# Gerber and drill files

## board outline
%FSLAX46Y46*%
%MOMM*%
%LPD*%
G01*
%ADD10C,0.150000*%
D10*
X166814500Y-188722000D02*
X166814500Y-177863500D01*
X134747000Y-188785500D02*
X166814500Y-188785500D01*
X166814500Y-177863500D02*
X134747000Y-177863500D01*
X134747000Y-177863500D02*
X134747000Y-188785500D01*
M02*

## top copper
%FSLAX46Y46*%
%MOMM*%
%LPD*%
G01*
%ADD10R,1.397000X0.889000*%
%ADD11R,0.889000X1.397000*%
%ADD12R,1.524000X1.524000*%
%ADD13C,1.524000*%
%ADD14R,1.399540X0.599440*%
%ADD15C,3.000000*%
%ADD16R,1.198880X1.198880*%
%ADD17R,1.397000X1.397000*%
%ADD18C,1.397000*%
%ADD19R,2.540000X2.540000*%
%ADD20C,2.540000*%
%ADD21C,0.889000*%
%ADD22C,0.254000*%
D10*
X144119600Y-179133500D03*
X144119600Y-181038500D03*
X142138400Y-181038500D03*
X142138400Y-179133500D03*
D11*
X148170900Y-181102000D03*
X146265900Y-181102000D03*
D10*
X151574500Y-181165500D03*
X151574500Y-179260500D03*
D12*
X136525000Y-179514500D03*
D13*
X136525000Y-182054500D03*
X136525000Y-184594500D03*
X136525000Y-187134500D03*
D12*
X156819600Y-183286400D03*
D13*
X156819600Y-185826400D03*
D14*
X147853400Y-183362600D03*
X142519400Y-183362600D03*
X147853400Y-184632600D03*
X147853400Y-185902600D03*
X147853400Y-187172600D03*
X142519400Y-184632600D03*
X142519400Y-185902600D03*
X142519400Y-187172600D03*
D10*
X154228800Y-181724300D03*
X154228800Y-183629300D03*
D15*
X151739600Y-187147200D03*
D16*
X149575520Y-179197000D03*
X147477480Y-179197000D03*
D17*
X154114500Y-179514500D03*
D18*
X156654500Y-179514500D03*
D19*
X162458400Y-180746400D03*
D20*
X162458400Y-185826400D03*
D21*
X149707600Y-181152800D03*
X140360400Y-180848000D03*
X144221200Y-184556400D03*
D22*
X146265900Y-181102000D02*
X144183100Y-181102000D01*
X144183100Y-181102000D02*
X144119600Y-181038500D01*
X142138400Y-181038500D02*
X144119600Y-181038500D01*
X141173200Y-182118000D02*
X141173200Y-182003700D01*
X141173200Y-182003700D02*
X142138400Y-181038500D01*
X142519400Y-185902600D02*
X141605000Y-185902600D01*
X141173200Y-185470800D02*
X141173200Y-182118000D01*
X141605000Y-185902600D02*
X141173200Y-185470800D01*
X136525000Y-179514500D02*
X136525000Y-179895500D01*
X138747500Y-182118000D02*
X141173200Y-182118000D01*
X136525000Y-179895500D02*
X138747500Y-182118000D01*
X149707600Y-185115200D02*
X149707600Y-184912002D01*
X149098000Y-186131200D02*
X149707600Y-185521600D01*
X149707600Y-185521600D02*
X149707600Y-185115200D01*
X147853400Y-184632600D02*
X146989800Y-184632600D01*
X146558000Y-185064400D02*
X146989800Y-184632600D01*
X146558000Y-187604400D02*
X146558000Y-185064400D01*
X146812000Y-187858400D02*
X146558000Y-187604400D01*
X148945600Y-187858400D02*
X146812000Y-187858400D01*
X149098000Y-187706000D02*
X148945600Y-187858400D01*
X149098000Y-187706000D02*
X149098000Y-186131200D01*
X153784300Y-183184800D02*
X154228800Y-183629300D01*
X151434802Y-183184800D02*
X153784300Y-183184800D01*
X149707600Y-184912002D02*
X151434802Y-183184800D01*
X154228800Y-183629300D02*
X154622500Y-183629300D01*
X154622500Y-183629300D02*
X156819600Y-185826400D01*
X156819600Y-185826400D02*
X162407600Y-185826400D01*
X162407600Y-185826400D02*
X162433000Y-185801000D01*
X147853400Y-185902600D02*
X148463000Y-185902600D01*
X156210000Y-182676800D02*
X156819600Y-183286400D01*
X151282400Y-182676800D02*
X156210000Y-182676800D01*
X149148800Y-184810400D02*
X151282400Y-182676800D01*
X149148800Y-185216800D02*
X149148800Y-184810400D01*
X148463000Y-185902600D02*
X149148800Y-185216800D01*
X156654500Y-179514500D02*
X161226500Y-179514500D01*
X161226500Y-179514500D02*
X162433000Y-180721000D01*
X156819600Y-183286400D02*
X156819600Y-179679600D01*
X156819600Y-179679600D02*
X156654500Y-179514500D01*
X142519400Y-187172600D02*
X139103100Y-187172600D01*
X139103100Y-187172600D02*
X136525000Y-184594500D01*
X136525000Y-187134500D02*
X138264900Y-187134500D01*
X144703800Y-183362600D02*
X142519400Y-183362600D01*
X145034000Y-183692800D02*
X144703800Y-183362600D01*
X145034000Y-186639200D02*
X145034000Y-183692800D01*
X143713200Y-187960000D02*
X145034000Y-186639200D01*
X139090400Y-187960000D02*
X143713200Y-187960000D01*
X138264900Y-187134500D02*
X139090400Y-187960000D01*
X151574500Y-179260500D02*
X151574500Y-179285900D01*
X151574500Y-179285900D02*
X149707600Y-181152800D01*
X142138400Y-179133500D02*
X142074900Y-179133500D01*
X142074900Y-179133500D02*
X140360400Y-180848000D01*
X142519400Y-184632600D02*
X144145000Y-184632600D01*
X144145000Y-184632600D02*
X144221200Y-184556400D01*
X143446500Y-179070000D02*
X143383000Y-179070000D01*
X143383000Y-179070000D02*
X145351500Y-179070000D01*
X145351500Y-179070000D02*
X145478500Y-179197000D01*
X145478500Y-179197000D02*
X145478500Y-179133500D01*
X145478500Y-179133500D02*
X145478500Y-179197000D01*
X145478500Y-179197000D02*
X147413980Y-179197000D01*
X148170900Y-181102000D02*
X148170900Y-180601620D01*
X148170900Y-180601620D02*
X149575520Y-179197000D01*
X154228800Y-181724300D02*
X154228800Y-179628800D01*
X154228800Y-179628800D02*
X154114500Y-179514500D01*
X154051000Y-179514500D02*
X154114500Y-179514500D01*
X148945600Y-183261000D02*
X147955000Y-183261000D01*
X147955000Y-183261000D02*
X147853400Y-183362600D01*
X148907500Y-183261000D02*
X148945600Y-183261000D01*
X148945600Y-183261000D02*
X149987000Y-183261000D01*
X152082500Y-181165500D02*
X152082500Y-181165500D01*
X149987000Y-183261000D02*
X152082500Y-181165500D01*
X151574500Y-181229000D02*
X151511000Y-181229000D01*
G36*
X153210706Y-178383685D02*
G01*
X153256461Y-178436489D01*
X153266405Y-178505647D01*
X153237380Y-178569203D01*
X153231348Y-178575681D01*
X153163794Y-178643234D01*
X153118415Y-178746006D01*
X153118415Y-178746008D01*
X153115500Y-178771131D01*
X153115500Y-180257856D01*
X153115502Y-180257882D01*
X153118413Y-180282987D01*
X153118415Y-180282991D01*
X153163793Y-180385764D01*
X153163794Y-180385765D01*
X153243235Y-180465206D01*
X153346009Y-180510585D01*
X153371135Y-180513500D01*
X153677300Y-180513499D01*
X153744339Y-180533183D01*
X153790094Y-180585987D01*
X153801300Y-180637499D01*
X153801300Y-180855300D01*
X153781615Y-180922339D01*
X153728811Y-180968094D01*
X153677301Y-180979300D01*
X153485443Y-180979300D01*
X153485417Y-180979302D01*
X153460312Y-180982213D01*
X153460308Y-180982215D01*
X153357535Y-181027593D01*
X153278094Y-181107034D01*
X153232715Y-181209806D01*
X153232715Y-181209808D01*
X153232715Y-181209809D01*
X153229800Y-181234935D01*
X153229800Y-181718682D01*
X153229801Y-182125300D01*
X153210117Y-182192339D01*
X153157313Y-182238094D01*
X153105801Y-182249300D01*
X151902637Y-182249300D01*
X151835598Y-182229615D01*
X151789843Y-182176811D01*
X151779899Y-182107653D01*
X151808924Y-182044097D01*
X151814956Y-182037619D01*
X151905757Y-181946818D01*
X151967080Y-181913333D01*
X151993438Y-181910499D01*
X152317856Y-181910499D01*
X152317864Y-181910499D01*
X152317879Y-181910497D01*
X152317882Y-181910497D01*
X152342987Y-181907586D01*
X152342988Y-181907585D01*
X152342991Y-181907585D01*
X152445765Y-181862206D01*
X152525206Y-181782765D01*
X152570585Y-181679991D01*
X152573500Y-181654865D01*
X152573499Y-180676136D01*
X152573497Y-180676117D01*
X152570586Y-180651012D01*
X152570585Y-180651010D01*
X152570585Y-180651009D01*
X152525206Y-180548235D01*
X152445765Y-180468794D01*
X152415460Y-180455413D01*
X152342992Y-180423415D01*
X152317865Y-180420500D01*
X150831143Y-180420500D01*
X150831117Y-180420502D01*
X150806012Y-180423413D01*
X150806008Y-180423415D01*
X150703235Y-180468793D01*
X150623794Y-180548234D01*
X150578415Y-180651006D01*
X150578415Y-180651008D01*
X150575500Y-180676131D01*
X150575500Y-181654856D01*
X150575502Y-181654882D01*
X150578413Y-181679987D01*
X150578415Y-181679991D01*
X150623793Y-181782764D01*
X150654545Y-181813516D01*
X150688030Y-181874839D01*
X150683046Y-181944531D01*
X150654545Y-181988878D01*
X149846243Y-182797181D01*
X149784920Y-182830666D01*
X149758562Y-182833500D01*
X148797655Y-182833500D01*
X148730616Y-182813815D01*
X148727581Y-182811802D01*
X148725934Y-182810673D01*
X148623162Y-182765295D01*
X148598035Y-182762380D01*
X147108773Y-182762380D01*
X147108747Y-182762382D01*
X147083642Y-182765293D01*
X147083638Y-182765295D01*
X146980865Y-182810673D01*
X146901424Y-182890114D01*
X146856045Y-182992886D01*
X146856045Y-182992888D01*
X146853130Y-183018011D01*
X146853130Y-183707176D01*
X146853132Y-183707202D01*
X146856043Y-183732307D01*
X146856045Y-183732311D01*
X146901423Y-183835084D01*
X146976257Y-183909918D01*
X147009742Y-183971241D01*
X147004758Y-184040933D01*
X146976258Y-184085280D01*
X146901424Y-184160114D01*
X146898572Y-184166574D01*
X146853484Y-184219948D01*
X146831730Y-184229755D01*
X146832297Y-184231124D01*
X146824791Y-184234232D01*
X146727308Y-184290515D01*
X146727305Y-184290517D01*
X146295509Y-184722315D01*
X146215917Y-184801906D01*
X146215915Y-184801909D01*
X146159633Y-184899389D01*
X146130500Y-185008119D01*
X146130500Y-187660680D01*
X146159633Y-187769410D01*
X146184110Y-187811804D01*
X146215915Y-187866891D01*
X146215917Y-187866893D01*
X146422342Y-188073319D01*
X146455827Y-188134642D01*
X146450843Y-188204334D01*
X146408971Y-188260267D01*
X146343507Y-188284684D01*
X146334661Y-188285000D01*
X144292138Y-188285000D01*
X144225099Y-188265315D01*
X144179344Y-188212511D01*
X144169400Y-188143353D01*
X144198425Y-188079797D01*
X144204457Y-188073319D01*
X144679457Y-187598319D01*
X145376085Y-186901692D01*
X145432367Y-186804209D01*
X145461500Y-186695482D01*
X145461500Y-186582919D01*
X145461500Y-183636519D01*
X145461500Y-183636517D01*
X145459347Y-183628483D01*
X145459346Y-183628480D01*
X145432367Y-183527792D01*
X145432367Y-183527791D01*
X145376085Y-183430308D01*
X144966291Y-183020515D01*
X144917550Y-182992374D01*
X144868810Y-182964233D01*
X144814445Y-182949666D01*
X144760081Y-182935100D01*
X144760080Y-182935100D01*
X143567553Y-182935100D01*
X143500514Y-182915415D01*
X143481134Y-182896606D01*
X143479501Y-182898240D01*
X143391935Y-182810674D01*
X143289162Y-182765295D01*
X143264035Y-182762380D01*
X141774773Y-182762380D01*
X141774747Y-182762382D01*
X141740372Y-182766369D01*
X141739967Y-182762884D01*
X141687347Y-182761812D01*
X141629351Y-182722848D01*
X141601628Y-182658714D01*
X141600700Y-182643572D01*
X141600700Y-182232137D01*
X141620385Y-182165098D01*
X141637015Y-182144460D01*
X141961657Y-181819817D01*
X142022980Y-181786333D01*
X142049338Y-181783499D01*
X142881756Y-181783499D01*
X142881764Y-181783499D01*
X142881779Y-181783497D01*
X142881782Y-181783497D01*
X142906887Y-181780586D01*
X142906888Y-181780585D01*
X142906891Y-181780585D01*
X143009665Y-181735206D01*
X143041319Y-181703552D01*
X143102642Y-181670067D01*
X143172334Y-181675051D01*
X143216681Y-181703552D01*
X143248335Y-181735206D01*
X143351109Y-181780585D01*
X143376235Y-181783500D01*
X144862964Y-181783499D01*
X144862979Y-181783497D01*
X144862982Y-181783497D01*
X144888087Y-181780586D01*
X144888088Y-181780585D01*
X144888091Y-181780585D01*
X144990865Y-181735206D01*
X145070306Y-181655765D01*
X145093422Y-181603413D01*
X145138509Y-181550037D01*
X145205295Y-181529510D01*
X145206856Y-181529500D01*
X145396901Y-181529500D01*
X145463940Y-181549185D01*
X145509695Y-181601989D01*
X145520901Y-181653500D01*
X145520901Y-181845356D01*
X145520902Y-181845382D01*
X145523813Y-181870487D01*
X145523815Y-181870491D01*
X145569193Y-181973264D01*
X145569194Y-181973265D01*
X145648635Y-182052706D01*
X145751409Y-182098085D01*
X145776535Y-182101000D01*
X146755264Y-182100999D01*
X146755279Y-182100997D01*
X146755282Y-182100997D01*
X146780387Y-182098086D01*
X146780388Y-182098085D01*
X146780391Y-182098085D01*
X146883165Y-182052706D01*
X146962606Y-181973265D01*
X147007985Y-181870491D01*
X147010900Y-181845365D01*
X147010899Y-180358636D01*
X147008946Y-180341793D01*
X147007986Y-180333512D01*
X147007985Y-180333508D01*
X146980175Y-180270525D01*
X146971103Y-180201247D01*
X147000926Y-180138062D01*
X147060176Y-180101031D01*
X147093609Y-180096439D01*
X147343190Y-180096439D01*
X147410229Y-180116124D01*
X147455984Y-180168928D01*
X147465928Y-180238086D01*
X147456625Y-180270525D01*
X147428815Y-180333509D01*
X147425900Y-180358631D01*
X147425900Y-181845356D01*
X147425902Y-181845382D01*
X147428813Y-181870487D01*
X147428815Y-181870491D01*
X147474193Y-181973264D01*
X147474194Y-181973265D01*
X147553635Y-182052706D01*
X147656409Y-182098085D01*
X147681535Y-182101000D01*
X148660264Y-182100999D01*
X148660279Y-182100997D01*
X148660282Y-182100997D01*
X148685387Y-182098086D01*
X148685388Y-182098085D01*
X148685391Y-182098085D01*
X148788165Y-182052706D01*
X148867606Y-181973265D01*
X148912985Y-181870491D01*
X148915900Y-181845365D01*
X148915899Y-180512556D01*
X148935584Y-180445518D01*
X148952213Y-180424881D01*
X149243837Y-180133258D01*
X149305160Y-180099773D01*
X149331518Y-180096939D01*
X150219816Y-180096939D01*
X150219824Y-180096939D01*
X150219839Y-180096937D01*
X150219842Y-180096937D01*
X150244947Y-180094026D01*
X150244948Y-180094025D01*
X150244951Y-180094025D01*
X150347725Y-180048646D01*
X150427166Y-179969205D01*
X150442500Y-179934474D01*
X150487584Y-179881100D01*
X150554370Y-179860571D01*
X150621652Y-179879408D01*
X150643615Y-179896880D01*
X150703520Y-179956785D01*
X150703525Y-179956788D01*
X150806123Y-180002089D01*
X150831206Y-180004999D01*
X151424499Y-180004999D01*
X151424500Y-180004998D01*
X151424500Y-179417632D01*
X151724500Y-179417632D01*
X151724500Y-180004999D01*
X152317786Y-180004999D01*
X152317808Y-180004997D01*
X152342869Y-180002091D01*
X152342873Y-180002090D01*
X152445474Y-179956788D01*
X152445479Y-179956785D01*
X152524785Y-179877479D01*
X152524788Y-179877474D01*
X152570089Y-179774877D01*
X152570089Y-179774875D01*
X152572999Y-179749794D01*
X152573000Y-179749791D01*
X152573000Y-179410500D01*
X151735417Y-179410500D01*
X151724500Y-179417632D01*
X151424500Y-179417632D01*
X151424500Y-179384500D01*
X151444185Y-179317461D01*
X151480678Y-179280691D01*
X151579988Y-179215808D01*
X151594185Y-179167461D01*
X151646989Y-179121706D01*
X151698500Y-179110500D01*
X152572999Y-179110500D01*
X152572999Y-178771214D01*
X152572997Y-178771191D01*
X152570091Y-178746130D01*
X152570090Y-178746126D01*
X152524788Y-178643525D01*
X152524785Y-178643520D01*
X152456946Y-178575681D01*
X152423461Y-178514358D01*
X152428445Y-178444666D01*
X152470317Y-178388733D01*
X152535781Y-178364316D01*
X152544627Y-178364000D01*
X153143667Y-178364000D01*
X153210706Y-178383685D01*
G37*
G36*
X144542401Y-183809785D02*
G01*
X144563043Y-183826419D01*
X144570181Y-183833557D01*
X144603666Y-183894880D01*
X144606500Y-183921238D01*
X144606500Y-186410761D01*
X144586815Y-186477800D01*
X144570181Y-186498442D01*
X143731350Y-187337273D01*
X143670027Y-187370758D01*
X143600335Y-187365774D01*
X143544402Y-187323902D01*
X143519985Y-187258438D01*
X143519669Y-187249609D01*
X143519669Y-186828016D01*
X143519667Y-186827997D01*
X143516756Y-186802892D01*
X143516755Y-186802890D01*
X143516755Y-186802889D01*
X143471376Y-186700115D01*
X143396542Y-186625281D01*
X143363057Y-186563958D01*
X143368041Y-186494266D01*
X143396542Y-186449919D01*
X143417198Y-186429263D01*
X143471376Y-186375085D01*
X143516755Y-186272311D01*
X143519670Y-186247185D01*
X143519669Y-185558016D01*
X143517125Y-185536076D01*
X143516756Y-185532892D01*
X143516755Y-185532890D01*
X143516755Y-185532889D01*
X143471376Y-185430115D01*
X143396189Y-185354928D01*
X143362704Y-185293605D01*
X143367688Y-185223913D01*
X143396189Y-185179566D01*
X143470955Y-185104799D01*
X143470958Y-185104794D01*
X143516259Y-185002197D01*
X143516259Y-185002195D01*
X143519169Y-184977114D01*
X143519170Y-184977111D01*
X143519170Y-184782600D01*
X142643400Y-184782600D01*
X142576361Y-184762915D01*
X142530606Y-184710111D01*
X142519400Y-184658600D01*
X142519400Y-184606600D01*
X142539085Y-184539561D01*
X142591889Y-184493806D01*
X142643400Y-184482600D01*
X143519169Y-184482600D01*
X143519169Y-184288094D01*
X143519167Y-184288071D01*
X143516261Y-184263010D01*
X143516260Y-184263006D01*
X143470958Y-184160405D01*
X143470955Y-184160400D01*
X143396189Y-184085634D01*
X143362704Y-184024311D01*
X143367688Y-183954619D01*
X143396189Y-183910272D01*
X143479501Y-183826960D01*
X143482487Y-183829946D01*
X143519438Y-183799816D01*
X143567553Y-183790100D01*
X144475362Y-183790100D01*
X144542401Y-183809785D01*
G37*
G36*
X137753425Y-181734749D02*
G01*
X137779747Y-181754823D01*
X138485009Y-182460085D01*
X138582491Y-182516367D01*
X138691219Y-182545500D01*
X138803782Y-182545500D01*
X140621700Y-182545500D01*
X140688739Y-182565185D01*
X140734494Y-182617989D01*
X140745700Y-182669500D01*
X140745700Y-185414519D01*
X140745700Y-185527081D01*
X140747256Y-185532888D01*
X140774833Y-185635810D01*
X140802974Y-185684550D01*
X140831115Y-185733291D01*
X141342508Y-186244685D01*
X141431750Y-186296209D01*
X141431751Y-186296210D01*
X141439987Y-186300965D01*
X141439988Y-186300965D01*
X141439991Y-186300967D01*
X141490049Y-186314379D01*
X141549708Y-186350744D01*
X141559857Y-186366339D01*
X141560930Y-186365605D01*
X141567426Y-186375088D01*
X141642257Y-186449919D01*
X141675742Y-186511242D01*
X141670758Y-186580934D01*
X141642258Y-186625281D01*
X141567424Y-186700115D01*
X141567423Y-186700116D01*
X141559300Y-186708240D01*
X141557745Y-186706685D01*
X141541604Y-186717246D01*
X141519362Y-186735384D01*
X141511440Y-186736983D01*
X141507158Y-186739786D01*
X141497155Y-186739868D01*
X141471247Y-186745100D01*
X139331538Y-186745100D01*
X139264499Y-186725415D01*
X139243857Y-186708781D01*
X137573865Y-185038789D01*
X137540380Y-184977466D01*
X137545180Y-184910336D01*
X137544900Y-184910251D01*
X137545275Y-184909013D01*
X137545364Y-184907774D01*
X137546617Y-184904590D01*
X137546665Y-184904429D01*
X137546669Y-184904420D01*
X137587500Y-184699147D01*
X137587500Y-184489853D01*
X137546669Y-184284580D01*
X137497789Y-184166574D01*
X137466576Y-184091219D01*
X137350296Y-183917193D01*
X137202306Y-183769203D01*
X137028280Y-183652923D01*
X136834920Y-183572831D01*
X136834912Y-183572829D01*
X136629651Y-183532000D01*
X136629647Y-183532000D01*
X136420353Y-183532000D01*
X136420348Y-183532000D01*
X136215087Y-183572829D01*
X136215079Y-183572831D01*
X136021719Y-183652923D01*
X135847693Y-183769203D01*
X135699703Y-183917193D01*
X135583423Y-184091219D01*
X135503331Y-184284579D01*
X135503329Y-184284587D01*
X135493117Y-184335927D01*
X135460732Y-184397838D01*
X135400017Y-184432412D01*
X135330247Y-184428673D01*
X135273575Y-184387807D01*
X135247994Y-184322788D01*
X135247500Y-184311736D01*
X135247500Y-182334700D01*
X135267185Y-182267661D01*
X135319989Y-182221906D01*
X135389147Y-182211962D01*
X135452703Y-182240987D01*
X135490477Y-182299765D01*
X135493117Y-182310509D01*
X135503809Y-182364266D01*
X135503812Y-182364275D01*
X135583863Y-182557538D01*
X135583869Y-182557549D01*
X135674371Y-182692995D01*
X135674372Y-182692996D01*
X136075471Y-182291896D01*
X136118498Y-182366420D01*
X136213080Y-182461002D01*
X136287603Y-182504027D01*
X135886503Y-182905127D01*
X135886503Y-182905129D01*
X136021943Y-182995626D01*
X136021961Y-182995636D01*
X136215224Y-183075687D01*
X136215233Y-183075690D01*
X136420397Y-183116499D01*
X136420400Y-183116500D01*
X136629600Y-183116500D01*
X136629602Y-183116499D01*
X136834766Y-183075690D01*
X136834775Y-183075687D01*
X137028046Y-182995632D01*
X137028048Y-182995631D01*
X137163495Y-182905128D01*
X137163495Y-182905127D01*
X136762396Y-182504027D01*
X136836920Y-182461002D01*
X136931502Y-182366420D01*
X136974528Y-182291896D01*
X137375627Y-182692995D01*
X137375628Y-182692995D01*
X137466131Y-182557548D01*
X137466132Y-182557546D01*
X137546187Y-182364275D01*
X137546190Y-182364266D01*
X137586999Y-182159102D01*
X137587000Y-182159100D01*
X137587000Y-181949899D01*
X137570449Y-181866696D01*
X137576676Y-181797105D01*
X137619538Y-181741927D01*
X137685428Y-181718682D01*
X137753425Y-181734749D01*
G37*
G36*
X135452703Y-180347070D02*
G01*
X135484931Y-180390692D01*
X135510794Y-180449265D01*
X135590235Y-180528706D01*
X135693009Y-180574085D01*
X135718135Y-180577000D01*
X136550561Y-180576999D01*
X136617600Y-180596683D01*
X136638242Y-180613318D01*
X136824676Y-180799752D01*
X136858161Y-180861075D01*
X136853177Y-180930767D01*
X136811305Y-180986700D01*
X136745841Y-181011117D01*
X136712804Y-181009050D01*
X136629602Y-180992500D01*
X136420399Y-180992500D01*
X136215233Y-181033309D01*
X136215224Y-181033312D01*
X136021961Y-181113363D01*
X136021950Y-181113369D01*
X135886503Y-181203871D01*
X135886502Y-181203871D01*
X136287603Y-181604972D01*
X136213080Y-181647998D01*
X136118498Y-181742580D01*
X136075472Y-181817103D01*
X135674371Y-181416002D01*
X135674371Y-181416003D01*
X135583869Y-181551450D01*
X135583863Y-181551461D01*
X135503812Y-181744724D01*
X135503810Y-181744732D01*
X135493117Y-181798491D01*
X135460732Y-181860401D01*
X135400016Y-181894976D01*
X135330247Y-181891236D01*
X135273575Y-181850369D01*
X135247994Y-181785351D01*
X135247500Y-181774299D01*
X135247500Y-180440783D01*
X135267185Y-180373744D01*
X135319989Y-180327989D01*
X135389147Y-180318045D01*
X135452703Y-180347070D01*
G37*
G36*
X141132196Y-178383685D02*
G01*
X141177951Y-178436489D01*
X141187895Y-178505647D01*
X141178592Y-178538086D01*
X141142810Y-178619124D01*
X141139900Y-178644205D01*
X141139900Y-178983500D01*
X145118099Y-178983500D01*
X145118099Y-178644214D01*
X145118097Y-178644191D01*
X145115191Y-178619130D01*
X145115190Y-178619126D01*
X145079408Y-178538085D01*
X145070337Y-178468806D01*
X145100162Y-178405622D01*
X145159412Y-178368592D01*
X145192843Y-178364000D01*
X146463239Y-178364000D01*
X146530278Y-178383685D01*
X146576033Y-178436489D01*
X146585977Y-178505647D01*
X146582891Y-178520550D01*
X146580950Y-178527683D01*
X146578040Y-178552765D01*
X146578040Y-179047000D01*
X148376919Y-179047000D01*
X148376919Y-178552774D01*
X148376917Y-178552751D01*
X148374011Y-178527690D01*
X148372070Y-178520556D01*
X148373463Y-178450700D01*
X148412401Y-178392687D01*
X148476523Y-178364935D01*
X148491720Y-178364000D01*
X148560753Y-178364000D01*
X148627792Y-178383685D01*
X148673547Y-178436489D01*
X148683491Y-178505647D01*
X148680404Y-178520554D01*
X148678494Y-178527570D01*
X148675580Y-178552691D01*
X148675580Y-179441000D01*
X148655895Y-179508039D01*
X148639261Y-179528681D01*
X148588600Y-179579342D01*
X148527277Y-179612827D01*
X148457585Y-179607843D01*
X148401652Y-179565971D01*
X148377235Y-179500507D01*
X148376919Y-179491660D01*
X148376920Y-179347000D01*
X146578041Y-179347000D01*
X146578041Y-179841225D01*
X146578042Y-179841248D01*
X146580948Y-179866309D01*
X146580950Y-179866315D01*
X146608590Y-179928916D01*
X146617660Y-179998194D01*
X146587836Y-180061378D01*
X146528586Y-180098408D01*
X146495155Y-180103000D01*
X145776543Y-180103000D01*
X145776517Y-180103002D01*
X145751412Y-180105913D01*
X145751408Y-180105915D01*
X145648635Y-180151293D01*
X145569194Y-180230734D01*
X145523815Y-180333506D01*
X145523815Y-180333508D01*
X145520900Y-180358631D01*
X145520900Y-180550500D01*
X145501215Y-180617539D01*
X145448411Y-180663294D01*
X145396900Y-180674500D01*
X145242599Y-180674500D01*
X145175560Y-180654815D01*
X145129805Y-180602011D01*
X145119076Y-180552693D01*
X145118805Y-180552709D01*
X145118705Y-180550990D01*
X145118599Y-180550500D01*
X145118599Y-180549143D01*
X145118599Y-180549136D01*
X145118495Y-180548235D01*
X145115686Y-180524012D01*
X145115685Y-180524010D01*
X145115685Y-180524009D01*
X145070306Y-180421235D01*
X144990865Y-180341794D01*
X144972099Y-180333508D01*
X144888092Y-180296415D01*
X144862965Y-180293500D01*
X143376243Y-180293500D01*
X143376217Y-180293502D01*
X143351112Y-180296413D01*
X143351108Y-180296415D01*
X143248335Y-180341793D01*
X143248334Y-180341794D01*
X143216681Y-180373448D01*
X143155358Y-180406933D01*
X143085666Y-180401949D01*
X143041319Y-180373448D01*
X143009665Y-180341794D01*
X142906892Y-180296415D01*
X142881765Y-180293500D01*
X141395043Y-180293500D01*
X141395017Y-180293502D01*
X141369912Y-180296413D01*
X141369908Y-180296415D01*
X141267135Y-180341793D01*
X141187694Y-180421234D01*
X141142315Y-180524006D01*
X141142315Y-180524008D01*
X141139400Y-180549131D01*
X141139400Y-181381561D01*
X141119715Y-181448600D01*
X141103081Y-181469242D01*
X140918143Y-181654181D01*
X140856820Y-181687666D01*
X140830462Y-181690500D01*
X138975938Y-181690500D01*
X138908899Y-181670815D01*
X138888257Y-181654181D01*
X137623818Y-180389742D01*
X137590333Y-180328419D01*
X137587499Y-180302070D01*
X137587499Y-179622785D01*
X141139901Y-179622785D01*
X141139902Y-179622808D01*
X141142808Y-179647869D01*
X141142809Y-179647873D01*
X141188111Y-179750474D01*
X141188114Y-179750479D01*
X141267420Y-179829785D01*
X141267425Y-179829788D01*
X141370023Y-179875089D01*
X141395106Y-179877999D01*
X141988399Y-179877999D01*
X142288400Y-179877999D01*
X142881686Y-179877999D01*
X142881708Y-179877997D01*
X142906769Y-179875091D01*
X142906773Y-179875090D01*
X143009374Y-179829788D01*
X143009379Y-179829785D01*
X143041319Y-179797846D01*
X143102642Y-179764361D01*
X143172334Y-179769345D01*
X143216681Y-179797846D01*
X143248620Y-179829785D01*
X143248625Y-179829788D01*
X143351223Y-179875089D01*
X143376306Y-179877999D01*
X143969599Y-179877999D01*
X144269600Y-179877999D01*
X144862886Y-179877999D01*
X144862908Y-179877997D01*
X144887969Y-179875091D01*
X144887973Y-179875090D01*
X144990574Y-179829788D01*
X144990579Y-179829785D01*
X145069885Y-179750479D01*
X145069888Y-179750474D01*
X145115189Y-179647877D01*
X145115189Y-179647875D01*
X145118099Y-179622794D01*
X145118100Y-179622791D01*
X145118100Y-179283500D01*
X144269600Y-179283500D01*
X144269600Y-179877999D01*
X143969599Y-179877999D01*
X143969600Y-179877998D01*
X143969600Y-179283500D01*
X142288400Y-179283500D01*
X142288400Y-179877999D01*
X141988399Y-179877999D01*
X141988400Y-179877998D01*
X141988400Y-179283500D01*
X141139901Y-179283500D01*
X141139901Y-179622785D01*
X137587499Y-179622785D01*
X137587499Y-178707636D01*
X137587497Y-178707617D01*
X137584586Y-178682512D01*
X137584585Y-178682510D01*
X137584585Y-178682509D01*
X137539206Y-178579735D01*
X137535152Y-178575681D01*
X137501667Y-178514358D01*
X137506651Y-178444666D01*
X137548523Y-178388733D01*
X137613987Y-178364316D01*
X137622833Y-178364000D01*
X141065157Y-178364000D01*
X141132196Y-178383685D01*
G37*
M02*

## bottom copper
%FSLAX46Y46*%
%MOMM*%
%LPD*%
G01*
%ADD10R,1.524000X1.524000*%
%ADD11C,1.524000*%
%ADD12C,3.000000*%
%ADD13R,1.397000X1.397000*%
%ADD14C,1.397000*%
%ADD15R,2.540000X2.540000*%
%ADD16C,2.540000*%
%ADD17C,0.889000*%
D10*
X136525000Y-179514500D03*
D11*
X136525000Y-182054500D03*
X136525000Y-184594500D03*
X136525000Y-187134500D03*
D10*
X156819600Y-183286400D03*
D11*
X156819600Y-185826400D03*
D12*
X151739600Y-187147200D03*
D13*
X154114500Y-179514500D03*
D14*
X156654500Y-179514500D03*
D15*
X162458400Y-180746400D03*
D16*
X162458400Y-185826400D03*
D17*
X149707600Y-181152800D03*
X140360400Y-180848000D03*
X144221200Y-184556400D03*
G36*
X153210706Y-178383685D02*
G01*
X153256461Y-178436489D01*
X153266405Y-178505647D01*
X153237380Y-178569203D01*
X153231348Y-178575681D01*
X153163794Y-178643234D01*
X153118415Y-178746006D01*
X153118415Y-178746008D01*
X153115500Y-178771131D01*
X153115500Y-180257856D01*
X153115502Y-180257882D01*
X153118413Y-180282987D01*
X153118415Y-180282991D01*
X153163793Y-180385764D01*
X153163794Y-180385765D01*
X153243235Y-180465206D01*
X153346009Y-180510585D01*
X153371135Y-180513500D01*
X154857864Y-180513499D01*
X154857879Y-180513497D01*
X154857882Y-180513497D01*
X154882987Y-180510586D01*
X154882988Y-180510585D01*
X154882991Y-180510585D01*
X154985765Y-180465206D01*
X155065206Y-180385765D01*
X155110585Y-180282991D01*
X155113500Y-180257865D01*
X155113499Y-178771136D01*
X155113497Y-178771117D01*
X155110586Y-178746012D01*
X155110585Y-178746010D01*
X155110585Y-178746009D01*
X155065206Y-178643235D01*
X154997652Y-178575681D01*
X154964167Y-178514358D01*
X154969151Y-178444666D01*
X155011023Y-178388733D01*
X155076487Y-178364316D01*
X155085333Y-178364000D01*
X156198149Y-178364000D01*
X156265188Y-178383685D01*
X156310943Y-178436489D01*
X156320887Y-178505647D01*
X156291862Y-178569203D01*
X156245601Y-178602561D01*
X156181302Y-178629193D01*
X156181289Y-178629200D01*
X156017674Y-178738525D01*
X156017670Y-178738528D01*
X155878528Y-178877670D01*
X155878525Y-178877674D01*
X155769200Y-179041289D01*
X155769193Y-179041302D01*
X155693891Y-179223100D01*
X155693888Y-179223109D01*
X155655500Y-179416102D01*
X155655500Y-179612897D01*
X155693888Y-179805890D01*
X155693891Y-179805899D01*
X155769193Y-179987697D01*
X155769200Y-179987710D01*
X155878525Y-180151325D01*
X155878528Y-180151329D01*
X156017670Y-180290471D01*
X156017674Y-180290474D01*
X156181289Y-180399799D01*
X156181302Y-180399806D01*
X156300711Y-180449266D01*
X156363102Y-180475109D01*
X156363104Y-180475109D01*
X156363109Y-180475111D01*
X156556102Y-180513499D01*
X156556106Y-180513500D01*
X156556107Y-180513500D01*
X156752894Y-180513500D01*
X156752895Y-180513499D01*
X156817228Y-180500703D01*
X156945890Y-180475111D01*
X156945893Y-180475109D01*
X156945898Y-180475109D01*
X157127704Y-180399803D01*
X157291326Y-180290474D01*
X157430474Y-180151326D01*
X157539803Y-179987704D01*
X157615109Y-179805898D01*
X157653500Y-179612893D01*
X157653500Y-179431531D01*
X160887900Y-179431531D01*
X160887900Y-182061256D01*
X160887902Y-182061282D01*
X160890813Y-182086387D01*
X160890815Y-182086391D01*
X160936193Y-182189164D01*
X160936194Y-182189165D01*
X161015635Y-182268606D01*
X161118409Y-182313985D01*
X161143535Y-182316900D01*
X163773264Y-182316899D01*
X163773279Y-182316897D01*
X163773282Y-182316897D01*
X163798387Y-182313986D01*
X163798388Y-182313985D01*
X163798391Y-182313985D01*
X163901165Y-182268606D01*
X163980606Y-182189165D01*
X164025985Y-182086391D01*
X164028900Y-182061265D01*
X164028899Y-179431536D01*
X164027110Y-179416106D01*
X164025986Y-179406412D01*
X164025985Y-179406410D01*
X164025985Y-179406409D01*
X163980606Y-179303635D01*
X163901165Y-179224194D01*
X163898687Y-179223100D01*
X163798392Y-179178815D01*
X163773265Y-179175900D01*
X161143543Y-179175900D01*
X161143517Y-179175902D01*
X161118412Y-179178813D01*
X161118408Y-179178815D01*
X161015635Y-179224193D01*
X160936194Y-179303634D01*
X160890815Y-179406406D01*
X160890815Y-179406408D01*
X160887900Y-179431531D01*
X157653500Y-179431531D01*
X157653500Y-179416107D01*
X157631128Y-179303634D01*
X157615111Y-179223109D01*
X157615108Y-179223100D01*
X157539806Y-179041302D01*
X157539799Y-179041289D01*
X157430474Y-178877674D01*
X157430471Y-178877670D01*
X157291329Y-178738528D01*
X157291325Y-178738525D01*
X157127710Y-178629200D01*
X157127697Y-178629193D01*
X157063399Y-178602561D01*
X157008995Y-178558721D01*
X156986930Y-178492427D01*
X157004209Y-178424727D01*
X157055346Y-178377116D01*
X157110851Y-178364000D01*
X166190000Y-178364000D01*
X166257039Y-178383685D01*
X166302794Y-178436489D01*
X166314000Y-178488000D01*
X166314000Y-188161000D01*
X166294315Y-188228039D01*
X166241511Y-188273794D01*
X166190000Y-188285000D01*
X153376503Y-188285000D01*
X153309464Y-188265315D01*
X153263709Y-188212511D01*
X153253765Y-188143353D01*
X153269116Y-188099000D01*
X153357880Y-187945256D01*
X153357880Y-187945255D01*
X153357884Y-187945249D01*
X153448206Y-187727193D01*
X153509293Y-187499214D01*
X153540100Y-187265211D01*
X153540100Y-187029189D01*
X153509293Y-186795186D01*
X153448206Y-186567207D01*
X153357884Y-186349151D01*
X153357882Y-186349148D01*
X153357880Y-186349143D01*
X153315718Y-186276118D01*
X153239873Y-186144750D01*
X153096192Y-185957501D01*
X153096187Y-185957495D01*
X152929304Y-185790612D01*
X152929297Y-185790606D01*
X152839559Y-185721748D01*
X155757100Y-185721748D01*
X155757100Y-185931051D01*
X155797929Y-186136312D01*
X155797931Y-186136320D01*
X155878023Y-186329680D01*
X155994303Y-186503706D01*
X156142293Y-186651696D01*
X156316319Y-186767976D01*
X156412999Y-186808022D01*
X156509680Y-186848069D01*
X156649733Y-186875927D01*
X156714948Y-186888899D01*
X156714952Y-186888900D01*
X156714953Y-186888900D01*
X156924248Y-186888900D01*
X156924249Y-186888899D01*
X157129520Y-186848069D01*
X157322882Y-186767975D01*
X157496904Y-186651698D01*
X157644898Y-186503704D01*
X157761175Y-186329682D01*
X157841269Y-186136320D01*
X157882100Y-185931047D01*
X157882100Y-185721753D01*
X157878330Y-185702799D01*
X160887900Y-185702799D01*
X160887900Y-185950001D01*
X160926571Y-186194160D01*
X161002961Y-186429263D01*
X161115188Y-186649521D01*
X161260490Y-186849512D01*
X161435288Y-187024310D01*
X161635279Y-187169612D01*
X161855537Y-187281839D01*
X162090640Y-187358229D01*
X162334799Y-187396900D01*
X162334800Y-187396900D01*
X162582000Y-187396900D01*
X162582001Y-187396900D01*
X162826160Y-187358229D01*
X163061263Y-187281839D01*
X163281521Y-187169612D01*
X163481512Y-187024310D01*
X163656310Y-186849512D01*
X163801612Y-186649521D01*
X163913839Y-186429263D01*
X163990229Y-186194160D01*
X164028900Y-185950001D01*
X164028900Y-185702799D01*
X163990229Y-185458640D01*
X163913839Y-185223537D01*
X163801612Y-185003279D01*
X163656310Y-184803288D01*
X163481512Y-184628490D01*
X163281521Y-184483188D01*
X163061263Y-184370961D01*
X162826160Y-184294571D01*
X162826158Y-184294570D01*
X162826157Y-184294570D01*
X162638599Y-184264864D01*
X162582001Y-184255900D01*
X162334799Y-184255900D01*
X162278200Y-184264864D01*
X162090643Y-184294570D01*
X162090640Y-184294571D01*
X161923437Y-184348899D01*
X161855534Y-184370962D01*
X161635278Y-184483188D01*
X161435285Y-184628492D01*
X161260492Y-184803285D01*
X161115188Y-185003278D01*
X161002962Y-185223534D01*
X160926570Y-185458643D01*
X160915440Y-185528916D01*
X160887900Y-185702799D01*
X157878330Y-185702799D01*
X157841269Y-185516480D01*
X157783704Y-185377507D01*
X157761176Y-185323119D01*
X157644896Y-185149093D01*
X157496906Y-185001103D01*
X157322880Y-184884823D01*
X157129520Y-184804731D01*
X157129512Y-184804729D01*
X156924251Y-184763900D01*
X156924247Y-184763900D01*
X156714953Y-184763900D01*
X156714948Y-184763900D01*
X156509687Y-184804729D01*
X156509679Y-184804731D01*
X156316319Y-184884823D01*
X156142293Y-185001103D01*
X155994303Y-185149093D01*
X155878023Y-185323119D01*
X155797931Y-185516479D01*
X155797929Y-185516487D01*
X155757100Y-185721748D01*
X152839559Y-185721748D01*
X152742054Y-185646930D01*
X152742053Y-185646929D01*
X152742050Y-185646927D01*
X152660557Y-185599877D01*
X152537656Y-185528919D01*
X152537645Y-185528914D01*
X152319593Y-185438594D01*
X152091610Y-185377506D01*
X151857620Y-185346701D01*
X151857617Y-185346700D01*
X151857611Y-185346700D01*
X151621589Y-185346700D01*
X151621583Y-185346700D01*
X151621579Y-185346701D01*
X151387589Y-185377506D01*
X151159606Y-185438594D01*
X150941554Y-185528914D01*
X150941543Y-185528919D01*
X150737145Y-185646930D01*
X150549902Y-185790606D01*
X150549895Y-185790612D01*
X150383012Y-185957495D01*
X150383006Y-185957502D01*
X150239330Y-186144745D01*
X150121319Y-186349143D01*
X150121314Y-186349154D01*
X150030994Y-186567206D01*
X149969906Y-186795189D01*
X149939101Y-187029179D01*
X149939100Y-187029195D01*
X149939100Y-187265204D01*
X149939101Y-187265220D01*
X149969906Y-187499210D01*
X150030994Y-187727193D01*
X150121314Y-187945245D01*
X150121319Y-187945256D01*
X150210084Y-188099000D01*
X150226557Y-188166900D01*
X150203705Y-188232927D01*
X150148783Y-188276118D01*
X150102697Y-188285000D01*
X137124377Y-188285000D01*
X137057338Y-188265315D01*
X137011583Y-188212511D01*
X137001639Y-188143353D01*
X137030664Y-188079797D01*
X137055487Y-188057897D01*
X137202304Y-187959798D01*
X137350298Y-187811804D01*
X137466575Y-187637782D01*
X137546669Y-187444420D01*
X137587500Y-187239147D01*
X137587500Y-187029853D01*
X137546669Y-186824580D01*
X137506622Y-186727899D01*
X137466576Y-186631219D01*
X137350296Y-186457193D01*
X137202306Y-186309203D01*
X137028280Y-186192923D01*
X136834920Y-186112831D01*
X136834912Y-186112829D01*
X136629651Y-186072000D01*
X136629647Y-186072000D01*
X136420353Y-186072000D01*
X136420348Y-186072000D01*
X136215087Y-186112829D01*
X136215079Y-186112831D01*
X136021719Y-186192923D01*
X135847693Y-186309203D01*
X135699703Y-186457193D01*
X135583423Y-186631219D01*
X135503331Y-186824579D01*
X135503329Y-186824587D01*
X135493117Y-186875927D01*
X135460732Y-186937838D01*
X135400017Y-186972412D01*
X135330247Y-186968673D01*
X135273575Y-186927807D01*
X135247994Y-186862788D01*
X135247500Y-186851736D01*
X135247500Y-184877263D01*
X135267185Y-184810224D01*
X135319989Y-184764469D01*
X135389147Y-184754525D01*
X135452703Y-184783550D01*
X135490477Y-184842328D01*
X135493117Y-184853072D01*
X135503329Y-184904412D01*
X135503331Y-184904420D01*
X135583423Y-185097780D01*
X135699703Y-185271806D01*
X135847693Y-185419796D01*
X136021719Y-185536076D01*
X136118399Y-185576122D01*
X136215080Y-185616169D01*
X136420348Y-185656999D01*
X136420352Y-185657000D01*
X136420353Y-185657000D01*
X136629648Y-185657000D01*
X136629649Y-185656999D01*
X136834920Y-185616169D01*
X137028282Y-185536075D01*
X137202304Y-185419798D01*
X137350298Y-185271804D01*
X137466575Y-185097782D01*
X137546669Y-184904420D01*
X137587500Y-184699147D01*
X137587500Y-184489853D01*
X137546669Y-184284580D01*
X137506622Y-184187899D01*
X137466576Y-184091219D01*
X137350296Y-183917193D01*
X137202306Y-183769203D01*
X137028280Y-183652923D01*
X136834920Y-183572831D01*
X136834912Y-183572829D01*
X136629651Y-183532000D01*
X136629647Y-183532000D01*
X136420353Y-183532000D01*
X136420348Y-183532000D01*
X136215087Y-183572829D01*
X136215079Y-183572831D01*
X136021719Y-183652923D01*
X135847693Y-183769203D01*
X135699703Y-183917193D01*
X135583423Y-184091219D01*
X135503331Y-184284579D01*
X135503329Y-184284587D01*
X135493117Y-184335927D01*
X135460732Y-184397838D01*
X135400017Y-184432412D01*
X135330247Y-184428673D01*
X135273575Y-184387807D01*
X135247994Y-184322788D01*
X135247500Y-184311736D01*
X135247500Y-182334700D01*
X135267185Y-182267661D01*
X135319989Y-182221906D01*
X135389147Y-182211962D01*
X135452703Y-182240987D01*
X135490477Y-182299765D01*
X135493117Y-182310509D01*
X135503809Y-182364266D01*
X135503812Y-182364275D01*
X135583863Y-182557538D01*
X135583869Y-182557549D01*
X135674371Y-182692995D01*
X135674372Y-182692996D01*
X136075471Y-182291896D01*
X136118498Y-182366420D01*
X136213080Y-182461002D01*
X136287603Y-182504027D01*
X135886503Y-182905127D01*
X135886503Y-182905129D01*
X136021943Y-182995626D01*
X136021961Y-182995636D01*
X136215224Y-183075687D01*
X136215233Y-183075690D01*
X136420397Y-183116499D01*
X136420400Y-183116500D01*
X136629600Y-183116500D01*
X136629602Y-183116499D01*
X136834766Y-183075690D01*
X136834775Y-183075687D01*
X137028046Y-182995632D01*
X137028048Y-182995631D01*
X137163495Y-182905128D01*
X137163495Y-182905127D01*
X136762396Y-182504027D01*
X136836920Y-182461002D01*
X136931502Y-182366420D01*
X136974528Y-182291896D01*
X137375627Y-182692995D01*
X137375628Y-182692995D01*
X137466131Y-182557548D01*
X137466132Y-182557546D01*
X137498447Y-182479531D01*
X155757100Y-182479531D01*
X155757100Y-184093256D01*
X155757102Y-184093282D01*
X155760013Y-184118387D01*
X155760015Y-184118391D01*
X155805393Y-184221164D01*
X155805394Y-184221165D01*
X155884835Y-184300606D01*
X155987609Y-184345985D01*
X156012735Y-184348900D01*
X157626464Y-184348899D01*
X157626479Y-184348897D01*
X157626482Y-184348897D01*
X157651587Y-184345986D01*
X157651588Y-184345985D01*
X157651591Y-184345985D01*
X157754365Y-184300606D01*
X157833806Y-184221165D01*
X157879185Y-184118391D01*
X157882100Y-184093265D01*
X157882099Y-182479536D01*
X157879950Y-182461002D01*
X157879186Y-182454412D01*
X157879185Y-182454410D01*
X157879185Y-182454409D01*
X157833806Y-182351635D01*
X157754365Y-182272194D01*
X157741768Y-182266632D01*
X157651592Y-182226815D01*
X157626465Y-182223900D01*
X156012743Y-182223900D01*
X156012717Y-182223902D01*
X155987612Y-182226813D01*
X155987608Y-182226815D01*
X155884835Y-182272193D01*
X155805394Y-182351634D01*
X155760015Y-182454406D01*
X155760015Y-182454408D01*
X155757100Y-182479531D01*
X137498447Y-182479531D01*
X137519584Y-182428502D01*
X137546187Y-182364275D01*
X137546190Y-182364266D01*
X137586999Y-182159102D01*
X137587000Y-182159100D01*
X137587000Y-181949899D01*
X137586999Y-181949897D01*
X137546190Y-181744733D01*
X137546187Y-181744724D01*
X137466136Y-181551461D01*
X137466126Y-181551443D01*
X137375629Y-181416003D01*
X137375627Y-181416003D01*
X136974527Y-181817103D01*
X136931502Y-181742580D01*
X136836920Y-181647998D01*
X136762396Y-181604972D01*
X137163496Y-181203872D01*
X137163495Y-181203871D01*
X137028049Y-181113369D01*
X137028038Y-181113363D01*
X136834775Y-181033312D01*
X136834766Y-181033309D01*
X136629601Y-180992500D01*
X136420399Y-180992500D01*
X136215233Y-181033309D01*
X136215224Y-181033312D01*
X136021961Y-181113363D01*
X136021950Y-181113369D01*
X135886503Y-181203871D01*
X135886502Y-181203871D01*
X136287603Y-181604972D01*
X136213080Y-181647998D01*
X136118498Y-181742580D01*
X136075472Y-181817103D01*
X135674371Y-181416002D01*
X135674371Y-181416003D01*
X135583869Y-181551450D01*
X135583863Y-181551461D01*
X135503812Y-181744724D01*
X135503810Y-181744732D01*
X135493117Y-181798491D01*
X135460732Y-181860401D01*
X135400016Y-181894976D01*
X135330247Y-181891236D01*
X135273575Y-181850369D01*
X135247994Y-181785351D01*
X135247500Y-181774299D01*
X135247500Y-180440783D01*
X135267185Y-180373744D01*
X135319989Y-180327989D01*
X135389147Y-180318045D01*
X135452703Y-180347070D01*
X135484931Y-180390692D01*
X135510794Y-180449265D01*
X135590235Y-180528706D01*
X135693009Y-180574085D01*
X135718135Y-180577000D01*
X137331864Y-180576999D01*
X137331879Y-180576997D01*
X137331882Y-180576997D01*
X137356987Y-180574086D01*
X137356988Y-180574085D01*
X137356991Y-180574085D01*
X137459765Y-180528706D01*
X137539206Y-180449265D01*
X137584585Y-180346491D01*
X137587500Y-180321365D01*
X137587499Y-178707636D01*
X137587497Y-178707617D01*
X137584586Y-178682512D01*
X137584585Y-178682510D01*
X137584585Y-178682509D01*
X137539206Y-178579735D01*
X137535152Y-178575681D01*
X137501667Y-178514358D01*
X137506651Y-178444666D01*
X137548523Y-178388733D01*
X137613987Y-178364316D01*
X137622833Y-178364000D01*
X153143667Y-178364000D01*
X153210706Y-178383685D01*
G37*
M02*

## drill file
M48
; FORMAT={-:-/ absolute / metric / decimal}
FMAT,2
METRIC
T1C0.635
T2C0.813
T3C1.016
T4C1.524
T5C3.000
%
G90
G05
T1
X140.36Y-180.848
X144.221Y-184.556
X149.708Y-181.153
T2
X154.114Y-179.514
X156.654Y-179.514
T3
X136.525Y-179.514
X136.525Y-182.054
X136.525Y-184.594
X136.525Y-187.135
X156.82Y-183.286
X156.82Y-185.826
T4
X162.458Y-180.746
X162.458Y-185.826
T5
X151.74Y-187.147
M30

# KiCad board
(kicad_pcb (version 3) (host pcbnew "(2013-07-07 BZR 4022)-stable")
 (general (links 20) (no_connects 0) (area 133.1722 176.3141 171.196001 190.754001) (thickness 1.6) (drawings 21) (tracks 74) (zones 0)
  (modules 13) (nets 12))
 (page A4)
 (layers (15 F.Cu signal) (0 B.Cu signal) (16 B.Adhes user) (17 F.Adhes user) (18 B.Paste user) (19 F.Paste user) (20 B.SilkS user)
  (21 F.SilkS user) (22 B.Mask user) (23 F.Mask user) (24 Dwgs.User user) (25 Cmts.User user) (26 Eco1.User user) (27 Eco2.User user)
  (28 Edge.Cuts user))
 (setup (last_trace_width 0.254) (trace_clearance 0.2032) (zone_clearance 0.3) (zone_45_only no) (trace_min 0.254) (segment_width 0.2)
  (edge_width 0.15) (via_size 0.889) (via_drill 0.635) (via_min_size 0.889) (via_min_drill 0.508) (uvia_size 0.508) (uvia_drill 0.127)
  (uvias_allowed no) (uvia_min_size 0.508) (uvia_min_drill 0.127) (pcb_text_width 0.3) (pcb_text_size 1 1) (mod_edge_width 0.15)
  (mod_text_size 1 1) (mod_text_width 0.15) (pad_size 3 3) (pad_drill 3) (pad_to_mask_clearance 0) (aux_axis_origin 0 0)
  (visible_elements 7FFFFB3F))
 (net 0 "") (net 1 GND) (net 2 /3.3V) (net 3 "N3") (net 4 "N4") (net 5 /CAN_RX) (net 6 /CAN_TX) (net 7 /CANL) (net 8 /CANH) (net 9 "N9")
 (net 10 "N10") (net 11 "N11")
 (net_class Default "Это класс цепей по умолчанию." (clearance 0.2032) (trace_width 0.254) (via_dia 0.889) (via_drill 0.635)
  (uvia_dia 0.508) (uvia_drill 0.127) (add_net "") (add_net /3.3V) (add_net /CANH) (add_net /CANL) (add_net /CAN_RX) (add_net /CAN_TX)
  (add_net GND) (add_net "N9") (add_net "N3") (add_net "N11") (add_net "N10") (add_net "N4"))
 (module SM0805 (layer F.Cu) (at 144.1196 180.086 270)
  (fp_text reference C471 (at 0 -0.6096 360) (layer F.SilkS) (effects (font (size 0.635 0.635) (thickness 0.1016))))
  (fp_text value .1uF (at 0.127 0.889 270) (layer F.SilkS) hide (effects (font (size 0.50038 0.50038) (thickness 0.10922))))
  (pad 1 smd rect (at -0.9525 0 270) (size 0.889 1.397) (layers F.Cu F.Paste F.Mask) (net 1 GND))
  (pad 2 smd rect (at 0.9525 0 270) (size 0.889 1.397) (layers F.Cu F.Paste F.Mask) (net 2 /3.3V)))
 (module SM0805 (layer F.Cu) (at 142.1384 180.086 90)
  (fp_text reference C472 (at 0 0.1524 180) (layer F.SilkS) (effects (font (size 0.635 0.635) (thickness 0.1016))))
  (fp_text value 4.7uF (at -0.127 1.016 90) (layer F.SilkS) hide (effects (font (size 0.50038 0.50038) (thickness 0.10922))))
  (pad 1 smd rect (at -0.9525 0 90) (size 0.889 1.397) (layers F.Cu F.Paste F.Mask) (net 2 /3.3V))
  (pad 2 smd rect (at 0.9525 0 90) (size 0.889 1.397) (layers F.Cu F.Paste F.Mask) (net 1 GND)))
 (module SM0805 (layer F.Cu) (at 147.2184 181.102 180)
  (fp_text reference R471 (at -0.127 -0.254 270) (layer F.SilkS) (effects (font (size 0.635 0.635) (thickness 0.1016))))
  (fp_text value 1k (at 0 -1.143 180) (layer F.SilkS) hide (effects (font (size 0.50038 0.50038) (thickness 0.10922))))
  (pad 1 smd rect (at -0.9525 0 180) (size 0.889 1.397) (layers F.Cu F.Paste F.Mask) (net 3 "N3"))
  (pad 2 smd rect (at 0.9525 0 180) (size 0.889 1.397) (layers F.Cu F.Paste F.Mask) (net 2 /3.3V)))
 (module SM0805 (layer F.Cu) (at 151.5745 180.213 90)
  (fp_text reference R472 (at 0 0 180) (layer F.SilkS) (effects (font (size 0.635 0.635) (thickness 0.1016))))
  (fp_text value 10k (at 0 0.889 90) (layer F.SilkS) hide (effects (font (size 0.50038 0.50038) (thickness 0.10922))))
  (pad 1 smd rect (at -0.9525 0 90) (size 0.889 1.397) (layers F.Cu F.Paste F.Mask) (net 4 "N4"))
  (pad 2 smd rect (at 0.9525 0 90) (size 0.889 1.397) (layers F.Cu F.Paste F.Mask) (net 1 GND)))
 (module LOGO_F (layer B.Cu) (at 146.4564 182.7784)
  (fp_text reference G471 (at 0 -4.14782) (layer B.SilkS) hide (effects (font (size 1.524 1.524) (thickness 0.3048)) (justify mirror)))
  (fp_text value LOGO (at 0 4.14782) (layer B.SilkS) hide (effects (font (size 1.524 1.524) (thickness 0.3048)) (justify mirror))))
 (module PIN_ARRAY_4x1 (layer F.Cu) (at 136.525 183.3245 270)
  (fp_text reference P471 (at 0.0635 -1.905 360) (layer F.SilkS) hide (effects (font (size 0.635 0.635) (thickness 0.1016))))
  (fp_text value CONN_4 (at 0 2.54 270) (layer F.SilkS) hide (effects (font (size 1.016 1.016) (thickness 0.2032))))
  (pad 1 thru_hole rect (at -3.81 0 270) (size 1.524 1.524) (drill 1.016) (layers *.Cu *.Mask F.SilkS) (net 2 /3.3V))
  (pad 2 thru_hole circle (at -1.27 0 270) (size 1.524 1.524) (drill 1.016) (layers *.Cu *.Mask F.SilkS) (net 1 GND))
  (pad 3 thru_hole circle (at 1.27 0 270) (size 1.524 1.524) (drill 1.016) (layers *.Cu *.Mask F.SilkS) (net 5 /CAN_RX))
  (pad 4 thru_hole circle (at 3.81 0 270) (size 1.524 1.524) (drill 1.016) (layers *.Cu *.Mask F.SilkS) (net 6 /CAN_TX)))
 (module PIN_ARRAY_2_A (layer F.Cu) (at 156.8196 184.5564 270)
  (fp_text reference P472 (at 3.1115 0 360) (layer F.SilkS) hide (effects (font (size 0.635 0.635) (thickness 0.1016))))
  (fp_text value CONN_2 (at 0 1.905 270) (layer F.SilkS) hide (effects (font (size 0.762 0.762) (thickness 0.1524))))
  (pad 1 thru_hole rect (at -1.27 0 270) (size 1.524 1.524) (drill 1.016) (layers *.Cu *.Mask F.SilkS) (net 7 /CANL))
  (pad 2 thru_hole circle (at 1.27 0 270) (size 1.524 1.524) (drill 1.016) (layers *.Cu *.Mask F.SilkS) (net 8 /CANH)))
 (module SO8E (layer F.Cu) (at 145.1864 185.2676 270)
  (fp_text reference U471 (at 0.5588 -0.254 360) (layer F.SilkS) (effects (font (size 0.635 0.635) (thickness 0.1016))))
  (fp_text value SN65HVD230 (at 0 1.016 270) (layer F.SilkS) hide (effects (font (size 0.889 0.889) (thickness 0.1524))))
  (pad 8 smd rect (at -1.905 -2.667 270) (size 0.59944 1.39954) (layers F.Cu F.Paste F.Mask) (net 4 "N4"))
  (pad 1 smd rect (at -1.905 2.667 270) (size 0.59944 1.39954) (layers F.Cu F.Paste F.Mask) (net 6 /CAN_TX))
  (pad 7 smd rect (at -0.635 -2.667 270) (size 0.59944 1.39954) (layers F.Cu F.Paste F.Mask) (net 8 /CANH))
  (pad 6 smd rect (at 0.635 -2.667 270) (size 0.59944 1.39954) (layers F.Cu F.Paste F.Mask) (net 7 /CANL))
  (pad 5 smd rect (at 1.905 -2.667 270) (size 0.59944 1.39954) (layers F.Cu F.Paste F.Mask) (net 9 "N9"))
  (pad 2 smd rect (at -0.635 2.667 270) (size 0.59944 1.39954) (layers F.Cu F.Paste F.Mask) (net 1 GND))
  (pad 3 smd rect (at 0.635 2.667 270) (size 0.59944 1.39954) (layers F.Cu F.Paste F.Mask) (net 2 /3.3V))
  (pad 4 smd rect (at 1.905 2.667 270) (size 0.59944 1.39954) (layers F.Cu F.Paste F.Mask) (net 5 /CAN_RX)))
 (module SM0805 (layer F.Cu) (at 154.2288 182.6768 270)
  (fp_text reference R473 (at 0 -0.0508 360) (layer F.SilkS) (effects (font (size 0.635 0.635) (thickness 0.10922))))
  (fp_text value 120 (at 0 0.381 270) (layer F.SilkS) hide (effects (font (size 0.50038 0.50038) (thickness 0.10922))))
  (pad 1 smd rect (at -0.9525 0 270) (size 0.889 1.397) (layers F.Cu F.Paste F.Mask) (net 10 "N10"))
  (pad 2 smd rect (at 0.9525 0 270) (size 0.889 1.397) (layers F.Cu F.Paste F.Mask) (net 8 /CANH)))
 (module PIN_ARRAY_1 (layer F.Cu) (at 151.7396 187.1472)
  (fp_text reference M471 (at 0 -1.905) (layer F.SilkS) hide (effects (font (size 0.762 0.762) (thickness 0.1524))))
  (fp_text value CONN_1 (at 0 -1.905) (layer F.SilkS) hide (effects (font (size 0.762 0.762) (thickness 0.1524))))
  (pad 1 thru_hole circle (at 0 0) (size 3 3) (drill 3) (layers *.Cu *.Mask F.SilkS) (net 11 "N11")))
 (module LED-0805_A (layer F.Cu) (at 148.5265 179.197 180)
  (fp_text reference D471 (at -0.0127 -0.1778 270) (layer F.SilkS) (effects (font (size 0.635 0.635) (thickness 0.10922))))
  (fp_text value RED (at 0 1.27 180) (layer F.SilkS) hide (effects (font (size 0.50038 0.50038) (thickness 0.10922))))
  (pad 1 smd rect (at -1.04902 0 180) (size 1.19888 1.19888) (layers F.Cu F.Paste F.Mask) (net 3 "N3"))
  (pad 2 smd rect (at 1.04902 0 180) (size 1.19888 1.19888) (layers F.Cu F.Paste F.Mask) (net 1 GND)))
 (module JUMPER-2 (layer F.Cu) (at 155.3845 179.5145)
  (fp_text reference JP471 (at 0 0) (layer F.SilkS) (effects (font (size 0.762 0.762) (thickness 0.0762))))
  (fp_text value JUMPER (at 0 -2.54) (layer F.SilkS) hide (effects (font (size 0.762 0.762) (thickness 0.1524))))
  (pad 1 thru_hole rect (at -1.27 0) (size 1.397 1.397) (drill 0.8128) (layers *.Cu *.Mask F.SilkS) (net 10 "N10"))
  (pad 2 thru_hole circle (at 1.27 0) (size 1.397 1.397) (drill 0.8128) (layers *.Cu *.Mask F.SilkS) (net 7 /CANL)))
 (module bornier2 (layer F.Cu) (at 162.4584 183.2864 270)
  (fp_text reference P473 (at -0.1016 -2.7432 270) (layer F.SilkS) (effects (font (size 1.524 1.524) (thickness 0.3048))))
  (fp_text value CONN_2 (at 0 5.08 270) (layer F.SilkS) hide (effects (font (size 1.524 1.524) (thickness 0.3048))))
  (pad 1 thru_hole rect (at -2.54 0 270) (size 2.54 2.54) (drill 1.524) (layers *.Cu *.Mask F.SilkS) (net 7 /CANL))
  (pad 2 thru_hole circle (at 2.54 0 270) (size 2.54 2.54) (drill 1.524) (layers *.Cu *.Mask F.SilkS) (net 8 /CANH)))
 (gr_line (start 166.8145 188.722) (end 166.8145 177.8635) (angle 90) (layer Edge.Cuts) (width 0.15))
 (gr_line (start 134.747 188.7855) (end 166.8145 188.7855) (angle 90) (layer Edge.Cuts) (width 0.15))
 (gr_line (start 166.8145 177.8635) (end 134.747 177.8635) (angle 90) (layer Edge.Cuts) (width 0.15))
 (gr_line (start 134.747 177.8635) (end 134.747 188.7855) (angle 90) (layer Edge.Cuts) (width 0.15))
 (segment (start 146.2659 181.102) (end 144.1831 181.102) (width 0.254) (layer F.Cu) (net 2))
 (segment (start 144.1831 181.102) (end 144.1196 181.0385) (width 0.254) (layer F.Cu) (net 2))
 (segment (start 142.1384 181.0385) (end 144.1196 181.0385) (width 0.254) (layer F.Cu) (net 2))
 (segment (start 141.1732 182.118) (end 141.1732 182.0037) (width 0.254) (layer F.Cu) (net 2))
 (segment (start 141.1732 182.0037) (end 142.1384 181.0385) (width 0.254) (layer F.Cu) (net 2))
 (segment (start 142.5194 185.9026) (end 141.605 185.9026) (width 0.254) (layer F.Cu) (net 2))
 (segment (start 141.1732 185.4708) (end 141.1732 182.118) (width 0.254) (layer F.Cu) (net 2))
 (segment (start 141.605 185.9026) (end 141.1732 185.4708) (width 0.254) (layer F.Cu) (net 2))
 (segment (start 136.525 179.5145) (end 136.525 179.8955) (width 0.254) (layer F.Cu) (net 2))
 (segment (start 138.7475 182.118) (end 141.1732 182.118) (width 0.254) (layer F.Cu) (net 2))
 (segment (start 136.525 179.8955) (end 138.7475 182.118) (width 0.254) (layer F.Cu) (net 2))
 (segment (start 149.7076 185.1152) (end 149.7076 184.912002) (width 0.254) (layer F.Cu) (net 8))
 (segment (start 149.098 186.1312) (end 149.7076 185.5216) (width 0.254) (layer F.Cu) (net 8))
 (segment (start 149.7076 185.5216) (end 149.7076 185.1152) (width 0.254) (layer F.Cu) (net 8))
 (segment (start 147.8534 184.6326) (end 146.9898 184.6326) (width 0.254) (layer F.Cu) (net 8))
 (segment (start 146.558 185.0644) (end 146.9898 184.6326) (width 0.254) (layer F.Cu) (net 8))
 (segment (start 146.558 187.6044) (end 146.558 185.0644) (width 0.254) (layer F.Cu) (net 8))
 (segment (start 146.812 187.8584) (end 146.558 187.6044) (width 0.254) (layer F.Cu) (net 8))
 (segment (start 148.9456 187.8584) (end 146.812 187.8584) (width 0.254) (layer F.Cu) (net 8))
 (segment (start 149.098 187.706) (end 148.9456 187.8584) (width 0.254) (layer F.Cu) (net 8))
 (segment (start 149.098 187.706) (end 149.098 186.1312) (width 0.254) (layer F.Cu) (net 8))
 (segment (start 153.7843 183.1848) (end 154.2288 183.6293) (width 0.254) (layer F.Cu) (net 8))
 (segment (start 151.434802 183.1848) (end 153.7843 183.1848) (width 0.254) (layer F.Cu) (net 8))
 (segment (start 149.7076 184.912002) (end 151.434802 183.1848) (width 0.254) (layer F.Cu) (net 8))
 (segment (start 154.2288 183.6293) (end 154.6225 183.6293) (width 0.254) (layer F.Cu) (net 8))
 (segment (start 154.6225 183.6293) (end 156.8196 185.8264) (width 0.254) (layer F.Cu) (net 8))
 (segment (start 156.8196 185.8264) (end 162.4076 185.8264) (width 0.254) (layer F.Cu) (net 8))
 (segment (start 162.4076 185.8264) (end 162.433 185.801) (width 0.254) (layer F.Cu) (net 8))
 (segment (start 147.8534 185.9026) (end 148.463 185.9026) (width 0.254) (layer F.Cu) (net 7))
 (segment (start 156.21 182.6768) (end 156.8196 183.2864) (width 0.254) (layer F.Cu) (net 7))
 (segment (start 151.2824 182.6768) (end 156.21 182.6768) (width 0.254) (layer F.Cu) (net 7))
 (segment (start 149.1488 184.8104) (end 151.2824 182.6768) (width 0.254) (layer F.Cu) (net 7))
 (segment (start 149.1488 185.2168) (end 149.1488 184.8104) (width 0.254) (layer F.Cu) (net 7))
 (segment (start 148.463 185.9026) (end 149.1488 185.2168) (width 0.254) (layer F.Cu) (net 7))
 (segment (start 156.6545 179.5145) (end 161.2265 179.5145) (width 0.254) (layer F.Cu) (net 7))
 (segment (start 161.2265 179.5145) (end 162.433 180.721) (width 0.254) (layer F.Cu) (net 7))
 (segment (start 156.8196 183.2864) (end 156.8196 179.6796) (width 0.254) (layer F.Cu) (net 7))
 (segment (start 156.8196 179.6796) (end 156.6545 179.5145) (width 0.254) (layer F.Cu) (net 7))
 (segment (start 142.5194 187.1726) (end 139.1031 187.1726) (width 0.254) (layer F.Cu) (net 5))
 (segment (start 139.1031 187.1726) (end 136.525 184.5945) (width 0.254) (layer F.Cu) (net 5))
 (segment (start 136.525 187.1345) (end 138.2649 187.1345) (width 0.254) (layer F.Cu) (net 6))
 (segment (start 144.7038 183.3626) (end 142.5194 183.3626) (width 0.254) (layer F.Cu) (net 6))
 (segment (start 145.034 183.6928) (end 144.7038 183.3626) (width 0.254) (layer F.Cu) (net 6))
 (segment (start 145.034 186.6392) (end 145.034 183.6928) (width 0.254) (layer F.Cu) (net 6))
 (segment (start 143.7132 187.96) (end 145.034 186.6392) (width 0.254) (layer F.Cu) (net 6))
 (segment (start 139.0904 187.96) (end 143.7132 187.96) (width 0.254) (layer F.Cu) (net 6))
 (segment (start 138.2649 187.1345) (end 139.0904 187.96) (width 0.254) (layer F.Cu) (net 6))
 (segment (start 151.5745 179.2605) (end 151.5745 179.2859) (width 0.254) (layer F.Cu) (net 1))
 (via (at 149.7076 181.1528) (size 0.889) (layers F.Cu B.Cu) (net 1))
 (segment (start 151.5745 179.2859) (end 149.7076 181.1528) (width 0.254) (layer F.Cu) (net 1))
 (segment (start 142.1384 179.1335) (end 142.0749 179.1335) (width 0.254) (layer F.Cu) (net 1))
 (via (at 140.3604 180.848) (size 0.889) (layers F.Cu B.Cu) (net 1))
 (segment (start 142.0749 179.1335) (end 140.3604 180.848) (width 0.254) (layer F.Cu) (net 1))
 (segment (start 142.5194 184.6326) (end 144.145 184.6326) (width 0.254) (layer F.Cu) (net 1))
 (via (at 144.2212 184.5564) (size 0.889) (layers F.Cu B.Cu) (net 1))
 (segment (start 144.145 184.6326) (end 144.2212 184.5564) (width 0.254) (layer F.Cu) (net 1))
 (segment (start 143.4465 179.07) (end 143.383 179.07) (width 0.254) (layer F.Cu) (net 1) (status 80000))
 (segment (start 143.383 179.07) (end 145.3515 179.07) (width 0.254) (layer F.Cu) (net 1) (status 80000))
 (segment (start 145.3515 179.07) (end 145.4785 179.197) (width 0.254) (layer F.Cu) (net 1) (status 80000))
 (segment (start 145.4785 179.197) (end 145.4785 179.1335) (width 0.254) (layer F.Cu) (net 1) (status 80000))
 (segment (start 145.4785 179.1335) (end 145.4785 179.197) (width 0.254) (layer F.Cu) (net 1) (status 80000))
 (segment (start 145.4785 179.197) (end 147.41398 179.197) (width 0.254) (layer F.Cu) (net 1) (status 80000))
 (segment (start 148.1709 181.102) (end 148.1709 180.60162) (width 0.254) (layer F.Cu) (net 3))
 (segment (start 148.1709 180.60162) (end 149.57552 179.197) (width 0.254) (layer F.Cu) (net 3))
 (segment (start 154.2288 181.7243) (end 154.2288 179.6288) (width 0.254) (layer F.Cu) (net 10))
 (segment (start 154.2288 179.6288) (end 154.1145 179.5145) (width 0.254) (layer F.Cu) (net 10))
 (segment (start 154.051 179.5145) (end 154.1145 179.5145) (width 0.254) (layer F.Cu) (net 10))
 (segment (start 148.9456 183.261) (end 147.955 183.261) (width 0.254) (layer F.Cu) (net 4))
 (segment (start 147.955 183.261) (end 147.8534 183.3626) (width 0.254) (layer F.Cu) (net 4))
 (segment (start 148.9075 183.261) (end 148.9456 183.261) (width 0.254) (layer F.Cu) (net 4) (status 10))
 (segment (start 148.9456 183.261) (end 149.987 183.261) (width 0.254) (layer F.Cu) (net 4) (status 10))
 (segment (start 152.0825 181.1655) (end 152.0825 181.1655) (width 0.254) (layer F.Cu) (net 4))
 (segment (start 149.987 183.261) (end 152.0825 181.1655) (width 0.254) (layer F.Cu) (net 4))
 (segment (start 151.5745 181.229) (end 151.511 181.229) (width 0.254) (layer F.Cu) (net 4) (status 80000))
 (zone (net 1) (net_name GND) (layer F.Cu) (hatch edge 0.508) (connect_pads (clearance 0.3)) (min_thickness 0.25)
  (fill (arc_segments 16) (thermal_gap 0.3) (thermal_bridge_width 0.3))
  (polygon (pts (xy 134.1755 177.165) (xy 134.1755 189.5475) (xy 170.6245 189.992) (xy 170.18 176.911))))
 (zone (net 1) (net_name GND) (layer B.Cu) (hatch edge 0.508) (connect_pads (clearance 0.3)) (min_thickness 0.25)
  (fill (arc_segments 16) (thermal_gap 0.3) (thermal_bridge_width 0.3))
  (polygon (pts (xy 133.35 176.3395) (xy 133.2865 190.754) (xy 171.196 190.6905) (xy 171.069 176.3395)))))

